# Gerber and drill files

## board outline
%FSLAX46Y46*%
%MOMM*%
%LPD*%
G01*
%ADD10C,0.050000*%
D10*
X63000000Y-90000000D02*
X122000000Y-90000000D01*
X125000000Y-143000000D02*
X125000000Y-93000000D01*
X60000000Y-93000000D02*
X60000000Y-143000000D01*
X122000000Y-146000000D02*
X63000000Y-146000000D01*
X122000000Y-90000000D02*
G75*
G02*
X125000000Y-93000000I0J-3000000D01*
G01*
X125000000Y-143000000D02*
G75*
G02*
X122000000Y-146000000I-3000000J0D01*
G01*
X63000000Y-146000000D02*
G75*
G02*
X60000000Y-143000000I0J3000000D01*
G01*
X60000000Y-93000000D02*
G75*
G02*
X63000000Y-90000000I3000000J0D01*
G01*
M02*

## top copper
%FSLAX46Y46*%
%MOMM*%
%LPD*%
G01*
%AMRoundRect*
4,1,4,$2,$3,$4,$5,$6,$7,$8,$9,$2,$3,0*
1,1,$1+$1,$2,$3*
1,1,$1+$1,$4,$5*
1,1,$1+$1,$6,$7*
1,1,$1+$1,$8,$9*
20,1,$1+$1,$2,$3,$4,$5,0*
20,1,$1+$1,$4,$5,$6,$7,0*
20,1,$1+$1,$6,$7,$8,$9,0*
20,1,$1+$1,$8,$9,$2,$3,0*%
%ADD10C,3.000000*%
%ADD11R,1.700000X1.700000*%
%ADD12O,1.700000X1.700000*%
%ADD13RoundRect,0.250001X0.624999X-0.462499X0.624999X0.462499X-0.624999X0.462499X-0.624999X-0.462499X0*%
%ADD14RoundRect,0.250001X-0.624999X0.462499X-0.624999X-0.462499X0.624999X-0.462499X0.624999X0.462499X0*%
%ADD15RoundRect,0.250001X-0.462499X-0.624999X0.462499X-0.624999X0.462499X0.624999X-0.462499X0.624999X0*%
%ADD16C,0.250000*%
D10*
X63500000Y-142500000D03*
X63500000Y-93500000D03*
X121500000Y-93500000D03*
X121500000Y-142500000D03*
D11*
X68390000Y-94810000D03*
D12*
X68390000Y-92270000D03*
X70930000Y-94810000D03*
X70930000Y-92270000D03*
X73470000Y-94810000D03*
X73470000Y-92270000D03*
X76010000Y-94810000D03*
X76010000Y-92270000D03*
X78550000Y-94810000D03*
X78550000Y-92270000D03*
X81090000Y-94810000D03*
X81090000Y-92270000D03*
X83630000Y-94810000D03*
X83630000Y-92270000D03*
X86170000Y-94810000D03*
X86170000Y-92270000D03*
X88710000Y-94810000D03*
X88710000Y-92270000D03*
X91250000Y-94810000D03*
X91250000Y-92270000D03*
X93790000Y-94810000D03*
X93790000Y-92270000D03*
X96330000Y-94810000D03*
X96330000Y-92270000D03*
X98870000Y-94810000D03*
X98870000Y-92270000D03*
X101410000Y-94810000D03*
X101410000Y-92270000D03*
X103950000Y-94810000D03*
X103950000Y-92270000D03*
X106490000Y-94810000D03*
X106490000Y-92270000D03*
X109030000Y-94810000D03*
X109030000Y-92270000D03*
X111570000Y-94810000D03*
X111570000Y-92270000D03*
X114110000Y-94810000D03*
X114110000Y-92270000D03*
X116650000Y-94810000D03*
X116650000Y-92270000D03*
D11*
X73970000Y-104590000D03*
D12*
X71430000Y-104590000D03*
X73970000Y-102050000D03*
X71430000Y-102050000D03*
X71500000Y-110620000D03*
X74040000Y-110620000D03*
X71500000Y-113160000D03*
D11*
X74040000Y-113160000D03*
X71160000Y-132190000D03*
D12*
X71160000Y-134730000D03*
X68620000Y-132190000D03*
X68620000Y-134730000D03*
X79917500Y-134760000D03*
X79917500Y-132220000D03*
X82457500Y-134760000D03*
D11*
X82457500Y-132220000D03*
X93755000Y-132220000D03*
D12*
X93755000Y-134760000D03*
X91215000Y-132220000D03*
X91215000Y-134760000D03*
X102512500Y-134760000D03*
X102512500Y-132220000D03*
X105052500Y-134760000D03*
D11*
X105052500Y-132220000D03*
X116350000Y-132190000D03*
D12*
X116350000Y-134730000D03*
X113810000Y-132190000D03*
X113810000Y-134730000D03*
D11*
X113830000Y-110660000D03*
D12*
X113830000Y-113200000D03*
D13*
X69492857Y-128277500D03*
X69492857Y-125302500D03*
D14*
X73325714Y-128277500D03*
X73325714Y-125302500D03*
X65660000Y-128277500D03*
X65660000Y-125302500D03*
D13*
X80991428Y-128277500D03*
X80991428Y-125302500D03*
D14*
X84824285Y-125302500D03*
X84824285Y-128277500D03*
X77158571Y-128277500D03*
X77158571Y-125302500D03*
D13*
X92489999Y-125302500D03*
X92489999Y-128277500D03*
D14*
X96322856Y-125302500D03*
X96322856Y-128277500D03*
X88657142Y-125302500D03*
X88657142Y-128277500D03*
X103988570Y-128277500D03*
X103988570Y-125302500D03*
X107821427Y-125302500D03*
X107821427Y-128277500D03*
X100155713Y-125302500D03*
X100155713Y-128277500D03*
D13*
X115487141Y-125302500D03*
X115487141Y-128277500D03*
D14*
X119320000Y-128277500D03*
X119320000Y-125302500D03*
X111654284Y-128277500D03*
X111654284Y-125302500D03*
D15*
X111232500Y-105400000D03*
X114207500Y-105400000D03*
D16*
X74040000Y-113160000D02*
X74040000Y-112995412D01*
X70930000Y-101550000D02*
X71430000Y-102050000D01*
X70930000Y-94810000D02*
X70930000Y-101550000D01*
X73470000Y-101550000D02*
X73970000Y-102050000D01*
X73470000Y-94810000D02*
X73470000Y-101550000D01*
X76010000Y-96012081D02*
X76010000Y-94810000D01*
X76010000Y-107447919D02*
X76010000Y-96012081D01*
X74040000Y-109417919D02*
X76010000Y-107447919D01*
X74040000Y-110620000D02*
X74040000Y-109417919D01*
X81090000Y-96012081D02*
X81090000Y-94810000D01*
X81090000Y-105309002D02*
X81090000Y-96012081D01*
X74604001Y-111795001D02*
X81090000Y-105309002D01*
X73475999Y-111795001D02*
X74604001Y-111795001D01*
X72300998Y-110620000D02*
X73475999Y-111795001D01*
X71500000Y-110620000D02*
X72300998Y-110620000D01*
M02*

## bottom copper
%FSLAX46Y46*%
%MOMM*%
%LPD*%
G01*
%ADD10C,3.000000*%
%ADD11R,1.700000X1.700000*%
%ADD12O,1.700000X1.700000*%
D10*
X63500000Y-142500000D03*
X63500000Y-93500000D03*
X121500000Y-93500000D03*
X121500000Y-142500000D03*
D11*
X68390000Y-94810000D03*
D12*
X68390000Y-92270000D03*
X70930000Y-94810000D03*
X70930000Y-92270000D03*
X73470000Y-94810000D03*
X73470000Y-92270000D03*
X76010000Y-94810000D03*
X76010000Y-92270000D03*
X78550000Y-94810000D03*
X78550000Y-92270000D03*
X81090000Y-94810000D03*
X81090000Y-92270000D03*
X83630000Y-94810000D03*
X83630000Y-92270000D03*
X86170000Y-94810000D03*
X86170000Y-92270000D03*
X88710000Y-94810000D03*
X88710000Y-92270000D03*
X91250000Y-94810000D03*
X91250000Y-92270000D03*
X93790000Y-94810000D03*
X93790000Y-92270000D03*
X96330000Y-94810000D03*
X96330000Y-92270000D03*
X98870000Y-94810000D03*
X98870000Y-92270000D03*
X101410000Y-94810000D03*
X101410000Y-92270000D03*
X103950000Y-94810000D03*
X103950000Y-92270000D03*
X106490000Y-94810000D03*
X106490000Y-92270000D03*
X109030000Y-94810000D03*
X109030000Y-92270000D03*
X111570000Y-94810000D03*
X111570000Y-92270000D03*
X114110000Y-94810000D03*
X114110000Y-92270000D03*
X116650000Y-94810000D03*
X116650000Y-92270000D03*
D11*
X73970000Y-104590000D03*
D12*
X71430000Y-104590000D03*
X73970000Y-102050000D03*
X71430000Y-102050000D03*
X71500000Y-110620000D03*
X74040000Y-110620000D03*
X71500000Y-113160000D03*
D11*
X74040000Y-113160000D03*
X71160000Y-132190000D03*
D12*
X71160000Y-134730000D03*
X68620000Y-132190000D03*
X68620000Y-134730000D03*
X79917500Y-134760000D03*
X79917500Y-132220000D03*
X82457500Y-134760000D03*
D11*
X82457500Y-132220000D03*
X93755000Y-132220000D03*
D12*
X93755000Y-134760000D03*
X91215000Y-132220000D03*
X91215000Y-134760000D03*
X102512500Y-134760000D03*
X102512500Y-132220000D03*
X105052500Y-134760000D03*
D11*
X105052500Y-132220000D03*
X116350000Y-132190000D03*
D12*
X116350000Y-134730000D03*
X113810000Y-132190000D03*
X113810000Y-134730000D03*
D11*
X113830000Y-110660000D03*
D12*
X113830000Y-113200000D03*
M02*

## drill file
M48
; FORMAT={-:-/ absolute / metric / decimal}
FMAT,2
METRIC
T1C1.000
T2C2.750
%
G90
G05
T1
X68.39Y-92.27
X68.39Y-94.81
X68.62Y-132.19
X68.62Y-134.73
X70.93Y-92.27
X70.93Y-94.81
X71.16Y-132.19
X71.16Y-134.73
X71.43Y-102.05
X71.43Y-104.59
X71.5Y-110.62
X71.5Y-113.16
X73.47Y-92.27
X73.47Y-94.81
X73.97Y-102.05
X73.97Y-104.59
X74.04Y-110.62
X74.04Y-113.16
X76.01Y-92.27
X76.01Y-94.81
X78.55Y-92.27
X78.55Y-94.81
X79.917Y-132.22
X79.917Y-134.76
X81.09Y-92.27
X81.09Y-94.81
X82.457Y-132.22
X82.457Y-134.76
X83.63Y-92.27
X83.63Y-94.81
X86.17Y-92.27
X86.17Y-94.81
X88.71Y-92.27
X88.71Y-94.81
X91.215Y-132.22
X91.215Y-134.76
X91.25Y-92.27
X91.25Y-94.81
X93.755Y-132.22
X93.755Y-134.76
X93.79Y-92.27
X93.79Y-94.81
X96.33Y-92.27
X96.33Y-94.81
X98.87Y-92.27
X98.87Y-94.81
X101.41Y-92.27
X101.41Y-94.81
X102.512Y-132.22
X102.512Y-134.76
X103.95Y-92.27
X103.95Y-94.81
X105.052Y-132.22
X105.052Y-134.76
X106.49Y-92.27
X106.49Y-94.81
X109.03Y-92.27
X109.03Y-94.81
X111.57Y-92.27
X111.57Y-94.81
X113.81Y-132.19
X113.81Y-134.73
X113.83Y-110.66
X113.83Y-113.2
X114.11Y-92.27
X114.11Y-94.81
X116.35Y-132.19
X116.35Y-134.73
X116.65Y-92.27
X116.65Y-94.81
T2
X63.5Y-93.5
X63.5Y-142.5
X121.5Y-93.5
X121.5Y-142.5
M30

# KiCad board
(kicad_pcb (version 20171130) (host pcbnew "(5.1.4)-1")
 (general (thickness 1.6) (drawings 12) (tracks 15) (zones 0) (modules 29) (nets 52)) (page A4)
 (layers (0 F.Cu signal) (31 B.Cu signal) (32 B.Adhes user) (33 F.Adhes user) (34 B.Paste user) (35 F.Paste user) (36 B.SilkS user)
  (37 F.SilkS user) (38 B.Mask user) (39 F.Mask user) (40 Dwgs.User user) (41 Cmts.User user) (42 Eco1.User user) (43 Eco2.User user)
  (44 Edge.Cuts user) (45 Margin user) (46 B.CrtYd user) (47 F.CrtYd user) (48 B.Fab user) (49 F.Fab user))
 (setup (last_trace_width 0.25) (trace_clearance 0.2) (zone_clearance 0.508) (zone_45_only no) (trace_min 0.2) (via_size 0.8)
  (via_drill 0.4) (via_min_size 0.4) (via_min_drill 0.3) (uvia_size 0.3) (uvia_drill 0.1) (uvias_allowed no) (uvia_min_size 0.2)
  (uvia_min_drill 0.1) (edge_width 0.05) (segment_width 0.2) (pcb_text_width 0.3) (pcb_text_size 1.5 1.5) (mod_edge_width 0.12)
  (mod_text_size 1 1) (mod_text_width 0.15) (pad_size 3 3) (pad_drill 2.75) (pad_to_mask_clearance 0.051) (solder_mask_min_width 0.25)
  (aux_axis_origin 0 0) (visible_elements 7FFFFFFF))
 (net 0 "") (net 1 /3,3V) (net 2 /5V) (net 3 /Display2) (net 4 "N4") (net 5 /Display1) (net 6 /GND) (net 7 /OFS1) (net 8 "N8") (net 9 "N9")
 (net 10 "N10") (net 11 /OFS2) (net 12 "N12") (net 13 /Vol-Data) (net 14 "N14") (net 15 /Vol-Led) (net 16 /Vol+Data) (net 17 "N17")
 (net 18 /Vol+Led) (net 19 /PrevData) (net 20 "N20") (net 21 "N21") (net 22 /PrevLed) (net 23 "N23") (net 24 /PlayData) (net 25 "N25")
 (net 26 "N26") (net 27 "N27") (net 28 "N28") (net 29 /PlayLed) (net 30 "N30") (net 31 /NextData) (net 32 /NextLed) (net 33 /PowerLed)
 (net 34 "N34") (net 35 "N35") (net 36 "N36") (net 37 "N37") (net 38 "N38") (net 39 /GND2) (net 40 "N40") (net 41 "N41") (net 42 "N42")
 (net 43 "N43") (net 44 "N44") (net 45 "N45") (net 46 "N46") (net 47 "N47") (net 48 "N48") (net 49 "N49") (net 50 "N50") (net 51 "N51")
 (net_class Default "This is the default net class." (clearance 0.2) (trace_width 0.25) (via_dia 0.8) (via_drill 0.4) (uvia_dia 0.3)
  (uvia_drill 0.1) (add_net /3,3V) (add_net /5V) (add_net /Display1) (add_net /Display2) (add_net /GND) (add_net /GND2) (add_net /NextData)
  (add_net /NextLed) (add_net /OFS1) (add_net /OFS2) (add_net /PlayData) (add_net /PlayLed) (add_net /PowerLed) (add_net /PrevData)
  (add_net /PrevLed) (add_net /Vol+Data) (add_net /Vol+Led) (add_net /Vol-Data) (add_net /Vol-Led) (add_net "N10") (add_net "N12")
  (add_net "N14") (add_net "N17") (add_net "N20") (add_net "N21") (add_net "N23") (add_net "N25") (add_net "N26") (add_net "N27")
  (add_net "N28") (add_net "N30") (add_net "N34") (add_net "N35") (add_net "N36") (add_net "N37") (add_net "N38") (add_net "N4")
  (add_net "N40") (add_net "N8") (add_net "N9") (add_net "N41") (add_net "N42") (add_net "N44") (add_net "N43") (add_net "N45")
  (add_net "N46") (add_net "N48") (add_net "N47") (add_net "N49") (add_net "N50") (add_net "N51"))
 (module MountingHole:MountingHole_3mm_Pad (layer F.Cu) (at 63.5 142.5)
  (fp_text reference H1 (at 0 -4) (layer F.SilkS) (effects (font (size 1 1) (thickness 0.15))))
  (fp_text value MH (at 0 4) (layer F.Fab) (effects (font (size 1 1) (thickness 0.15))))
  (pad "" np_thru_hole circle (at 0 0) (size 3 3) (drill 2.75) (layers *.Cu *.Mask)))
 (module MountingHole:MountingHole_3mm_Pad (layer F.Cu) (at 63.5 93.5)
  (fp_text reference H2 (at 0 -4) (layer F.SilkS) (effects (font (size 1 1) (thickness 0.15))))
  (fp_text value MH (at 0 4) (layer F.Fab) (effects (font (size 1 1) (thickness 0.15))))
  (pad "" np_thru_hole circle (at 0 0) (size 3 3) (drill 2.75) (layers *.Cu *.Mask)))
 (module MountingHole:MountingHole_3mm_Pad (layer F.Cu) (at 121.5 93.5)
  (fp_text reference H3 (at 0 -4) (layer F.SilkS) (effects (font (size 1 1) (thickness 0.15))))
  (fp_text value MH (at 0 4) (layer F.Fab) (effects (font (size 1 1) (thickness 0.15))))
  (pad "" np_thru_hole circle (at 0 0) (size 3 3) (drill 2.75) (layers *.Cu *.Mask)))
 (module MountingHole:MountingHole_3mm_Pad (layer F.Cu) (at 121.5 142.5)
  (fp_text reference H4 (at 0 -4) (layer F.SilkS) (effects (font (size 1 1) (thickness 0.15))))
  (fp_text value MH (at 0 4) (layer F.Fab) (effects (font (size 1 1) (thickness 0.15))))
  (pad "" np_thru_hole circle (at 0 0) (size 3 3) (drill 2.75) (layers *.Cu *.Mask)))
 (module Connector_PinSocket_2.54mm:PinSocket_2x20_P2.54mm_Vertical (layer B.Cu) (at 68.39 94.81 270)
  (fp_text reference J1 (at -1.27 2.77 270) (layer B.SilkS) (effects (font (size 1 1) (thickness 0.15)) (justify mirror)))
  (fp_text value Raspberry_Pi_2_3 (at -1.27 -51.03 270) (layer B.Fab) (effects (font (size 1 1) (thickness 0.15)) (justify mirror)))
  (pad 1 thru_hole rect (at 0 0 270) (size 1.7 1.7) (drill 1) (layers *.Cu *.Mask) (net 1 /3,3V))
  (pad 2 thru_hole oval (at -2.54 0 270) (size 1.7 1.7) (drill 1) (layers *.Cu *.Mask) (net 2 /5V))
  (pad 3 thru_hole oval (at 0 -2.54 270) (size 1.7 1.7) (drill 1) (layers *.Cu *.Mask) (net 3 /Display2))
  (pad 4 thru_hole oval (at -2.54 -2.54 270) (size 1.7 1.7) (drill 1) (layers *.Cu *.Mask) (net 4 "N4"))
  (pad 5 thru_hole oval (at 0 -5.08 270) (size 1.7 1.7) (drill 1) (layers *.Cu *.Mask) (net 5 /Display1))
  (pad 6 thru_hole oval (at -2.54 -5.08 270) (size 1.7 1.7) (drill 1) (layers *.Cu *.Mask) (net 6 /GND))
  (pad 7 thru_hole oval (at 0 -7.62 270) (size 1.7 1.7) (drill 1) (layers *.Cu *.Mask) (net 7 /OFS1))
  (pad 8 thru_hole oval (at -2.54 -7.62 270) (size 1.7 1.7) (drill 1) (layers *.Cu *.Mask) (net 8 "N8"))
  (pad 9 thru_hole oval (at 0 -10.16 270) (size 1.7 1.7) (drill 1) (layers *.Cu *.Mask) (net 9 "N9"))
  (pad 10 thru_hole oval (at -2.54 -10.16 270) (size 1.7 1.7) (drill 1) (layers *.Cu *.Mask) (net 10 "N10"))
  (pad 11 thru_hole oval (at 0 -12.7 270) (size 1.7 1.7) (drill 1) (layers *.Cu *.Mask) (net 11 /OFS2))
  (pad 12 thru_hole oval (at -2.54 -12.7 270) (size 1.7 1.7) (drill 1) (layers *.Cu *.Mask) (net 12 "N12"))
  (pad 13 thru_hole oval (at 0 -15.24 270) (size 1.7 1.7) (drill 1) (layers *.Cu *.Mask) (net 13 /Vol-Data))
  (pad 14 thru_hole oval (at -2.54 -15.24 270) (size 1.7 1.7) (drill 1) (layers *.Cu *.Mask) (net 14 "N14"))
  (pad 15 thru_hole oval (at 0 -17.78 270) (size 1.7 1.7) (drill 1) (layers *.Cu *.Mask) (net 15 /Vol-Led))
  (pad 16 thru_hole oval (at -2.54 -17.78 270) (size 1.7 1.7) (drill 1) (layers *.Cu *.Mask) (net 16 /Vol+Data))
  (pad 17 thru_hole oval (at 0 -20.32 270) (size 1.7 1.7) (drill 1) (layers *.Cu *.Mask) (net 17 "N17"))
  (pad 18 thru_hole oval (at -2.54 -20.32 270) (size 1.7 1.7) (drill 1) (layers *.Cu *.Mask) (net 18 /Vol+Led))
  (pad 19 thru_hole oval (at 0 -22.86 270) (size 1.7 1.7) (drill 1) (layers *.Cu *.Mask) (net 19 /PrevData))
  (pad 20 thru_hole oval (at -2.54 -22.86 270) (size 1.7 1.7) (drill 1) (layers *.Cu *.Mask) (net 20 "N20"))
  (pad 21 thru_hole oval (at 0 -25.4 270) (size 1.7 1.7) (drill 1) (layers *.Cu *.Mask) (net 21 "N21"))
  (pad 22 thru_hole oval (at -2.54 -25.4 270) (size 1.7 1.7) (drill 1) (layers *.Cu *.Mask) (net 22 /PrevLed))
  (pad 23 thru_hole oval (at 0 -27.94 270) (size 1.7 1.7) (drill 1) (layers *.Cu *.Mask) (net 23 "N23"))
  (pad 24 thru_hole oval (at -2.54 -27.94 270) (size 1.7 1.7) (drill 1) (layers *.Cu *.Mask) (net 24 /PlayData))
  (pad 25 thru_hole oval (at 0 -30.48 270) (size 1.7 1.7) (drill 1) (layers *.Cu *.Mask) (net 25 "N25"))
  (pad 26 thru_hole oval (at -2.54 -30.48 270) (size 1.7 1.7) (drill 1) (layers *.Cu *.Mask) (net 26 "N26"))
  (pad 27 thru_hole oval (at 0 -33.02 270) (size 1.7 1.7) (drill 1) (layers *.Cu *.Mask) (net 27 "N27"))
  (pad 28 thru_hole oval (at -2.54 -33.02 270) (size 1.7 1.7) (drill 1) (layers *.Cu *.Mask) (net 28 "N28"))
  (pad 29 thru_hole oval (at 0 -35.56 270) (size 1.7 1.7) (drill 1) (layers *.Cu *.Mask) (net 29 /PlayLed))
  (pad 30 thru_hole oval (at -2.54 -35.56 270) (size 1.7 1.7) (drill 1) (layers *.Cu *.Mask) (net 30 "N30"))
  (pad 31 thru_hole oval (at 0 -38.1 270) (size 1.7 1.7) (drill 1) (layers *.Cu *.Mask) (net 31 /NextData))
  (pad 32 thru_hole oval (at -2.54 -38.1 270) (size 1.7 1.7) (drill 1) (layers *.Cu *.Mask) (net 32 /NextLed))
  (pad 33 thru_hole oval (at 0 -40.64 270) (size 1.7 1.7) (drill 1) (layers *.Cu *.Mask) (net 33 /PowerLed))
  (pad 34 thru_hole oval (at -2.54 -40.64 270) (size 1.7 1.7) (drill 1) (layers *.Cu *.Mask) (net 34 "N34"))
  (pad 35 thru_hole oval (at 0 -43.18 270) (size 1.7 1.7) (drill 1) (layers *.Cu *.Mask) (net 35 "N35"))
  (pad 36 thru_hole oval (at -2.54 -43.18 270) (size 1.7 1.7) (drill 1) (layers *.Cu *.Mask) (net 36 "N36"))
  (pad 37 thru_hole oval (at 0 -45.72 270) (size 1.7 1.7) (drill 1) (layers *.Cu *.Mask) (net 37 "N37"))
  (pad 38 thru_hole oval (at -2.54 -45.72 270) (size 1.7 1.7) (drill 1) (layers *.Cu *.Mask) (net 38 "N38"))
  (pad 39 thru_hole oval (at 0 -48.26 270) (size 1.7 1.7) (drill 1) (layers *.Cu *.Mask) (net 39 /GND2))
  (pad 40 thru_hole oval (at -2.54 -48.26 270) (size 1.7 1.7) (drill 1) (layers *.Cu *.Mask) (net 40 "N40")))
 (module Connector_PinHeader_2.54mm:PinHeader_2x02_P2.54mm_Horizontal (layer F.Cu) (at 73.97 104.59 180)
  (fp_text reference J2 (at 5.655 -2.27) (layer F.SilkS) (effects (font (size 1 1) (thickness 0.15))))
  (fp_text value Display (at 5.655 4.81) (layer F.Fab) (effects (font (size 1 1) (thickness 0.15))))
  (pad 1 thru_hole rect (at 0 0 180) (size 1.7 1.7) (drill 1) (layers *.Cu *.Mask) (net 2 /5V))
  (pad 2 thru_hole oval (at 2.54 0 180) (size 1.7 1.7) (drill 1) (layers *.Cu *.Mask) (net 6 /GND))
  (pad 3 thru_hole oval (at 0 2.54 180) (size 1.7 1.7) (drill 1) (layers *.Cu *.Mask) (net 5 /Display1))
  (pad 4 thru_hole oval (at 2.54 2.54 180) (size 1.7 1.7) (drill 1) (layers *.Cu *.Mask) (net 3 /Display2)))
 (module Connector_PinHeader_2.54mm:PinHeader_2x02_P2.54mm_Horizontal (layer F.Cu) (at 74.04 113.16 180)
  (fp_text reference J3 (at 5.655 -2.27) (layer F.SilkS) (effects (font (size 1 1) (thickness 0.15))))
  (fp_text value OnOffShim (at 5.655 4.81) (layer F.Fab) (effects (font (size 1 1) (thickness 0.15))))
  (pad 4 thru_hole oval (at 2.54 2.54 180) (size 1.7 1.7) (drill 1) (layers *.Cu *.Mask) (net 11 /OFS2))
  (pad 3 thru_hole oval (at 0 2.54 180) (size 1.7 1.7) (drill 1) (layers *.Cu *.Mask) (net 7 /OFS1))
  (pad 2 thru_hole oval (at 2.54 0 180) (size 1.7 1.7) (drill 1) (layers *.Cu *.Mask) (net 6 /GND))
  (pad 1 thru_hole rect (at 0 0 180) (size 1.7 1.7) (drill 1) (layers *.Cu *.Mask) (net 2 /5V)))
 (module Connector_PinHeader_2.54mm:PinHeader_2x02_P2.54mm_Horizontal (layer F.Cu) (at 71.16 132.19 270)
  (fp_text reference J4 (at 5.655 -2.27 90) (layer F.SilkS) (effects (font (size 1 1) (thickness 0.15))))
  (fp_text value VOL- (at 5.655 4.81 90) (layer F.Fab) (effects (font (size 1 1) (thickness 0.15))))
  (pad 1 thru_hole rect (at 0 0 270) (size 1.7 1.7) (drill 1) (layers *.Cu *.Mask) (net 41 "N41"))
  (pad 2 thru_hole oval (at 2.54 0 270) (size 1.7 1.7) (drill 1) (layers *.Cu *.Mask) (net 6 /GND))
  (pad 3 thru_hole oval (at 0 2.54 270) (size 1.7 1.7) (drill 1) (layers *.Cu *.Mask) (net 6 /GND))
  (pad 4 thru_hole oval (at 2.54 2.54 270) (size 1.7 1.7) (drill 1) (layers *.Cu *.Mask) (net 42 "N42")))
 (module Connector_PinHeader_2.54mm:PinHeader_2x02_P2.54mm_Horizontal (layer F.Cu) (at 82.4575 132.22 270)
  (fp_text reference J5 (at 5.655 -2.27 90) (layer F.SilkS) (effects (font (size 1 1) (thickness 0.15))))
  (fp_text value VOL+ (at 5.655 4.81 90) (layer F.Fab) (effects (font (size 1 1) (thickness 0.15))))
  (pad 4 thru_hole oval (at 2.54 2.54 270) (size 1.7 1.7) (drill 1) (layers *.Cu *.Mask) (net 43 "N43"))
  (pad 3 thru_hole oval (at 0 2.54 270) (size 1.7 1.7) (drill 1) (layers *.Cu *.Mask) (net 6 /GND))
  (pad 2 thru_hole oval (at 2.54 0 270) (size 1.7 1.7) (drill 1) (layers *.Cu *.Mask) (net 6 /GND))
  (pad 1 thru_hole rect (at 0 0 270) (size 1.7 1.7) (drill 1) (layers *.Cu *.Mask) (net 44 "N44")))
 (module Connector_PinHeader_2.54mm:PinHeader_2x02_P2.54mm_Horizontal (layer F.Cu) (at 93.755 132.22 270)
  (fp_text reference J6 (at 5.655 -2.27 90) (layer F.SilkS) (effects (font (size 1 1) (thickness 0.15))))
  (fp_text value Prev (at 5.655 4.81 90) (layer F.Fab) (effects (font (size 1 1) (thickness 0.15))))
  (pad 1 thru_hole rect (at 0 0 270) (size 1.7 1.7) (drill 1) (layers *.Cu *.Mask) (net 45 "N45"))
  (pad 2 thru_hole oval (at 2.54 0 270) (size 1.7 1.7) (drill 1) (layers *.Cu *.Mask) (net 39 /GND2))
  (pad 3 thru_hole oval (at 0 2.54 270) (size 1.7 1.7) (drill 1) (layers *.Cu *.Mask) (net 39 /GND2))
  (pad 4 thru_hole oval (at 2.54 2.54 270) (size 1.7 1.7) (drill 1) (layers *.Cu *.Mask) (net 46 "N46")))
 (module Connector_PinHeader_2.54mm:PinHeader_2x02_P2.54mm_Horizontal (layer F.Cu) (at 105.0525 132.22 270)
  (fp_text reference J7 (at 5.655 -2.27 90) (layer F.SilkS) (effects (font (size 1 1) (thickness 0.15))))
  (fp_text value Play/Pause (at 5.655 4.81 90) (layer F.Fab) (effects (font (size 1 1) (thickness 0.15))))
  (pad 4 thru_hole oval (at 2.54 2.54 270) (size 1.7 1.7) (drill 1) (layers *.Cu *.Mask) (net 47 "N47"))
  (pad 3 thru_hole oval (at 0 2.54 270) (size 1.7 1.7) (drill 1) (layers *.Cu *.Mask) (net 39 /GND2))
  (pad 2 thru_hole oval (at 2.54 0 270) (size 1.7 1.7) (drill 1) (layers *.Cu *.Mask) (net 39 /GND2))
  (pad 1 thru_hole rect (at 0 0 270) (size 1.7 1.7) (drill 1) (layers *.Cu *.Mask) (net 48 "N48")))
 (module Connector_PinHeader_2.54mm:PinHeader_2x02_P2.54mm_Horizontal (layer F.Cu) (at 116.35 132.19 270)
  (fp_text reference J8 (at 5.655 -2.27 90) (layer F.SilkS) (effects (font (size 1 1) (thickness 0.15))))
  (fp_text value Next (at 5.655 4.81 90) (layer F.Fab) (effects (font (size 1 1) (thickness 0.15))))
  (pad 1 thru_hole rect (at 0 0 270) (size 1.7 1.7) (drill 1) (layers *.Cu *.Mask) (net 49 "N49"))
  (pad 2 thru_hole oval (at 2.54 0 270) (size 1.7 1.7) (drill 1) (layers *.Cu *.Mask) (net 39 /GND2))
  (pad 3 thru_hole oval (at 0 2.54 270) (size 1.7 1.7) (drill 1) (layers *.Cu *.Mask) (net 39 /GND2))
  (pad 4 thru_hole oval (at 2.54 2.54 270) (size 1.7 1.7) (drill 1) (layers *.Cu *.Mask) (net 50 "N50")))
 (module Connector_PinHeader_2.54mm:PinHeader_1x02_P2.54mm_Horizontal (layer F.Cu) (at 113.83 110.66)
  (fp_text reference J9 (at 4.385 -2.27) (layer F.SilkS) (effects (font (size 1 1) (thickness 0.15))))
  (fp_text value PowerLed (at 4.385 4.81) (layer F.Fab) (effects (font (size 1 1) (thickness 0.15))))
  (pad 1 thru_hole rect (at 0 0) (size 1.7 1.7) (drill 1) (layers *.Cu *.Mask) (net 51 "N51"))
  (pad 2 thru_hole oval (at 0 2.54) (size 1.7 1.7) (drill 1) (layers *.Cu *.Mask) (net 39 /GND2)))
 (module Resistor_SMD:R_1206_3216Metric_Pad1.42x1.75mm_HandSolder (layer F.Cu) (at 69.492857 126.79 90)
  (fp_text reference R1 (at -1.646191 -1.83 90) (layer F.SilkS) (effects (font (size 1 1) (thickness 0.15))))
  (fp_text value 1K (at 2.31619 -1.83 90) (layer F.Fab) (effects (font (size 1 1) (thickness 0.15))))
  (pad 1 smd roundrect (at -1.4875 0 90) (size 1.425 1.75) (layers F.Cu F.Paste F.Mask) (roundrect_rratio 0.175439) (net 41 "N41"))
  (pad 2 smd roundrect (at 1.4875 0 90) (size 1.425 1.75) (layers F.Cu F.Paste F.Mask) (roundrect_rratio 0.175439) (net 13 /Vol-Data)))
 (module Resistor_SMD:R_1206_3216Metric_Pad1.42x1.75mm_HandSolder (layer F.Cu) (at 73.325714 126.79 270)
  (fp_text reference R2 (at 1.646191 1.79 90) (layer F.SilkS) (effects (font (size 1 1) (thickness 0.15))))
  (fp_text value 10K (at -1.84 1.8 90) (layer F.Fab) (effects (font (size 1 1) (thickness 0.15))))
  (pad 2 smd roundrect (at 1.4875 0 270) (size 1.425 1.75) (layers F.Cu F.Paste F.Mask) (roundrect_rratio 0.175439) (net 41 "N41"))
  (pad 1 smd roundrect (at -1.4875 0 270) (size 1.425 1.75) (layers F.Cu F.Paste F.Mask) (roundrect_rratio 0.175439) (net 1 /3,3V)))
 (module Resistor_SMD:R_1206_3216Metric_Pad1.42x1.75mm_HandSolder (layer F.Cu) (at 65.66 126.79 270)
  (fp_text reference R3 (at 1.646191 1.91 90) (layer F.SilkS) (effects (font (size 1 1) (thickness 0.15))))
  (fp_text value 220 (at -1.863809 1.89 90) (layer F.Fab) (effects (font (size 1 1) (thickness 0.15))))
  (pad 2 smd roundrect (at 1.4875 0 270) (size 1.425 1.75) (layers F.Cu F.Paste F.Mask) (roundrect_rratio 0.175439) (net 42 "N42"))
  (pad 1 smd roundrect (at -1.4875 0 270) (size 1.425 1.75) (layers F.Cu F.Paste F.Mask) (roundrect_rratio 0.175439) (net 15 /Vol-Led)))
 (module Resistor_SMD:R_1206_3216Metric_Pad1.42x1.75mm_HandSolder (layer F.Cu) (at 80.991428 126.79 90)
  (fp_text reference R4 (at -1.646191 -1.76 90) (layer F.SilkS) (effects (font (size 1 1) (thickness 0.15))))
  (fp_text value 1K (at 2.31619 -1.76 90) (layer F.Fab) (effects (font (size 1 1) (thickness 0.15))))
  (pad 1 smd roundrect (at -1.4875 0 90) (size 1.425 1.75) (layers F.Cu F.Paste F.Mask) (roundrect_rratio 0.175439) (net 44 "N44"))
  (pad 2 smd roundrect (at 1.4875 0 90) (size 1.425 1.75) (layers F.Cu F.Paste F.Mask) (roundrect_rratio 0.175439) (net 16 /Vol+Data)))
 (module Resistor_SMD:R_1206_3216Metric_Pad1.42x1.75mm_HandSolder (layer F.Cu) (at 84.824285 126.79 270)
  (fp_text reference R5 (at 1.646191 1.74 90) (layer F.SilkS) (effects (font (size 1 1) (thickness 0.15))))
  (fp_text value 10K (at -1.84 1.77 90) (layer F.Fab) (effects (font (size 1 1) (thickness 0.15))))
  (pad 1 smd roundrect (at -1.4875 0 270) (size 1.425 1.75) (layers F.Cu F.Paste F.Mask) (roundrect_rratio 0.175439) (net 1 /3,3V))
  (pad 2 smd roundrect (at 1.4875 0 270) (size 1.425 1.75) (layers F.Cu F.Paste F.Mask) (roundrect_rratio 0.175439) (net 44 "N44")))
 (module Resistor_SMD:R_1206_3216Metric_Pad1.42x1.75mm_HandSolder (layer F.Cu) (at 77.158571 126.79 270)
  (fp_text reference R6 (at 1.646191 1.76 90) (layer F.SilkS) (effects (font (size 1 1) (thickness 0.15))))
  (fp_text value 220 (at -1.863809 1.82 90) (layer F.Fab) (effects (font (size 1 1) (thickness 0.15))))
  (pad 2 smd roundrect (at 1.4875 0 270) (size 1.425 1.75) (layers F.Cu F.Paste F.Mask) (roundrect_rratio 0.175439) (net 43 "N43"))
  (pad 1 smd roundrect (at -1.4875 0 270) (size 1.425 1.75) (layers F.Cu F.Paste F.Mask) (roundrect_rratio 0.175439) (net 18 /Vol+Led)))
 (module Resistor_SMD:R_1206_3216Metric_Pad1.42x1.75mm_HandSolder (layer F.Cu) (at 92.489999 126.79 90)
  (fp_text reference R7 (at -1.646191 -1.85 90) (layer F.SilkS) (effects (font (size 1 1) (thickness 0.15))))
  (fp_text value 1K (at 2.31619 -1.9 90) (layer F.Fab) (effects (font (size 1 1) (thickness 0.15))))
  (pad 2 smd roundrect (at 1.4875 0 90) (size 1.425 1.75) (layers F.Cu F.Paste F.Mask) (roundrect_rratio 0.175439) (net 19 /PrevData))
  (pad 1 smd roundrect (at -1.4875 0 90) (size 1.425 1.75) (layers F.Cu F.Paste F.Mask) (roundrect_rratio 0.175439) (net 45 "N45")))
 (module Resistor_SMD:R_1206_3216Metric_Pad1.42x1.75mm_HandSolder (layer F.Cu) (at 96.322856 126.79 270)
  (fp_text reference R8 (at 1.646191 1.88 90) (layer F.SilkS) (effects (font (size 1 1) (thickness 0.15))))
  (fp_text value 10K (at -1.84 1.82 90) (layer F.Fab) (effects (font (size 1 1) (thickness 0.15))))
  (pad 1 smd roundrect (at -1.4875 0 270) (size 1.425 1.75) (layers F.Cu F.Paste F.Mask) (roundrect_rratio 0.175439) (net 1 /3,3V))
  (pad 2 smd roundrect (at 1.4875 0 270) (size 1.425 1.75) (layers F.Cu F.Paste F.Mask) (roundrect_rratio 0.175439) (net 45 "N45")))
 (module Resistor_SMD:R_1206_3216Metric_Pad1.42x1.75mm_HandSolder (layer F.Cu) (at 88.657142 126.79 270)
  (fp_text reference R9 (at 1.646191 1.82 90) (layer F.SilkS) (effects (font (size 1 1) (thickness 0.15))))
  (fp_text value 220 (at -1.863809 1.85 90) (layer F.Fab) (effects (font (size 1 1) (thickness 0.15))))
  (pad 1 smd roundrect (at -1.4875 0 270) (size 1.425 1.75) (layers F.Cu F.Paste F.Mask) (roundrect_rratio 0.175439) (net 22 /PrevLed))
  (pad 2 smd roundrect (at 1.4875 0 270) (size 1.425 1.75) (layers F.Cu F.Paste F.Mask) (roundrect_rratio 0.175439) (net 46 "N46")))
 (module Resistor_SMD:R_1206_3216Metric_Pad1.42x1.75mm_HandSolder (layer F.Cu) (at 103.98857 126.79 270)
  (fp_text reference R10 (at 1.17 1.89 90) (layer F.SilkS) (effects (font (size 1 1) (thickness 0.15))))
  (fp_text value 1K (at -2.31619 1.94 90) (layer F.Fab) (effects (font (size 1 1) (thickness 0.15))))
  (pad 2 smd roundrect (at 1.4875 0 270) (size 1.425 1.75) (layers F.Cu F.Paste F.Mask) (roundrect_rratio 0.175439) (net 24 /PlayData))
  (pad 1 smd roundrect (at -1.4875 0 270) (size 1.425 1.75) (layers F.Cu F.Paste F.Mask) (roundrect_rratio 0.175439) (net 48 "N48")))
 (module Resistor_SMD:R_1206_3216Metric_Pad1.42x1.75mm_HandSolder (layer F.Cu) (at 107.821427 126.79 270)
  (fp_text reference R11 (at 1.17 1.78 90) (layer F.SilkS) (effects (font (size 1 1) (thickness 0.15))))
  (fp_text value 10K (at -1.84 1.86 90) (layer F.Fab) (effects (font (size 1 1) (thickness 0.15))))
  (pad 1 smd roundrect (at -1.4875 0 270) (size 1.425 1.75) (layers F.Cu F.Paste F.Mask) (roundrect_rratio 0.175439) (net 1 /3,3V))
  (pad 2 smd roundrect (at 1.4875 0 270) (size 1.425 1.75) (layers F.Cu F.Paste F.Mask) (roundrect_rratio 0.175439) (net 48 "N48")))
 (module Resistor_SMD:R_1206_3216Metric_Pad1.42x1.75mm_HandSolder (layer F.Cu) (at 100.155713 126.79 270)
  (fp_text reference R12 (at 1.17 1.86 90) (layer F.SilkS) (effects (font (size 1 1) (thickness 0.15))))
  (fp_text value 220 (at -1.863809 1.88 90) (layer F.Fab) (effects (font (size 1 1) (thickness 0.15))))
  (pad 1 smd roundrect (at -1.4875 0 270) (size 1.425 1.75) (layers F.Cu F.Paste F.Mask) (roundrect_rratio 0.175439) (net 29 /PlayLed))
  (pad 2 smd roundrect (at 1.4875 0 270) (size 1.425 1.75) (layers F.Cu F.Paste F.Mask) (roundrect_rratio 0.175439) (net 47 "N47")))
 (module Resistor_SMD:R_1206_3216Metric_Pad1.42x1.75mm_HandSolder (layer F.Cu) (at 115.487141 126.79 90)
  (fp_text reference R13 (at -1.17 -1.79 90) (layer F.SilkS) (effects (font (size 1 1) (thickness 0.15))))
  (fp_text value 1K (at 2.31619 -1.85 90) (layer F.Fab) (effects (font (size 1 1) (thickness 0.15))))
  (pad 2 smd roundrect (at 1.4875 0 90) (size 1.425 1.75) (layers F.Cu F.Paste F.Mask) (roundrect_rratio 0.175439) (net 31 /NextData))
  (pad 1 smd roundrect (at -1.4875 0 90) (size 1.425 1.75) (layers F.Cu F.Paste F.Mask) (roundrect_rratio 0.175439) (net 49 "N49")))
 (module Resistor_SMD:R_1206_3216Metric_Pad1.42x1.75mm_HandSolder (layer F.Cu) (at 119.32 126.79 270)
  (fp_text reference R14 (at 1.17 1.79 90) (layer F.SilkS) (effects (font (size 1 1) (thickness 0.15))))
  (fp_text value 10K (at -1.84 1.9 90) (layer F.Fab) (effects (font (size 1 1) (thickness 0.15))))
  (pad 2 smd roundrect (at 1.4875 0 270) (size 1.425 1.75) (layers F.Cu F.Paste F.Mask) (roundrect_rratio 0.175439) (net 49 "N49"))
  (pad 1 smd roundrect (at -1.4875 0 270) (size 1.425 1.75) (layers F.Cu F.Paste F.Mask) (roundrect_rratio 0.175439) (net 1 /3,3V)))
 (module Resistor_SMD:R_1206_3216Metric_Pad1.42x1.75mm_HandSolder (layer F.Cu) (at 111.654284 126.79 270)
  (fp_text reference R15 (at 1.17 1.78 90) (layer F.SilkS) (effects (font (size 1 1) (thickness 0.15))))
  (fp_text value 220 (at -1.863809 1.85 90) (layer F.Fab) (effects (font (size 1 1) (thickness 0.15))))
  (pad 2 smd roundrect (at 1.4875 0 270) (size 1.425 1.75) (layers F.Cu F.Paste F.Mask) (roundrect_rratio 0.175439) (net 50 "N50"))
  (pad 1 smd roundrect (at -1.4875 0 270) (size 1.425 1.75) (layers F.Cu F.Paste F.Mask) (roundrect_rratio 0.175439) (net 32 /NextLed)))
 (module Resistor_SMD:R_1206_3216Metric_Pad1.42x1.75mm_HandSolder (layer F.Cu) (at 112.72 105.4)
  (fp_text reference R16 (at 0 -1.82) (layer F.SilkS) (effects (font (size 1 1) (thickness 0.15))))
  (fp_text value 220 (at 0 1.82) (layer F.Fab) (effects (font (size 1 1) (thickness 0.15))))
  (pad 1 smd roundrect (at -1.4875 0) (size 1.425 1.75) (layers F.Cu F.Paste F.Mask) (roundrect_rratio 0.175439) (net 33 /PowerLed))
  (pad 2 smd roundrect (at 1.4875 0) (size 1.425 1.75) (layers F.Cu F.Paste F.Mask) (roundrect_rratio 0.175439) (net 51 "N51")))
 (gr_line (start 63 90) (end 122 90) (layer Edge.Cuts) (width 0.05))
 (gr_line (start 125 143) (end 125 93) (layer Edge.Cuts) (width 0.05))
 (gr_line (start 60 93) (end 60 143) (layer Edge.Cuts) (width 0.05))
 (gr_line (start 122 146) (end 63 146) (layer Edge.Cuts) (width 0.05))
 (gr_arc (start 122 93) (end 125 93) (angle -90) (layer Edge.Cuts) (width 0.05))
 (gr_arc (start 122 143) (end 122 146) (angle -90) (layer Edge.Cuts) (width 0.05))
 (gr_arc (start 63 143) (end 60 143) (angle -90) (layer Edge.Cuts) (width 0.05))
 (gr_arc (start 63 93) (end 63 90) (angle -90) (layer Edge.Cuts) (width 0.05))
 (segment (start 74.04 113.16) (end 74.04 112.995412) (width 0.25) (layer F.Cu) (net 2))
 (segment (start 70.93 101.55) (end 71.43 102.05) (width 0.25) (layer F.Cu) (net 3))
 (segment (start 70.93 94.81) (end 70.93 101.55) (width 0.25) (layer F.Cu) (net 3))
 (segment (start 73.47 101.55) (end 73.97 102.05) (width 0.25) (layer F.Cu) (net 5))
 (segment (start 73.47 94.81) (end 73.47 101.55) (width 0.25) (layer F.Cu) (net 5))
 (segment (start 76.01 96.012081) (end 76.01 94.81) (width 0.25) (layer F.Cu) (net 7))
 (segment (start 76.01 107.447919) (end 76.01 96.012081) (width 0.25) (layer F.Cu) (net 7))
 (segment (start 74.04 109.417919) (end 76.01 107.447919) (width 0.25) (layer F.Cu) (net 7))
 (segment (start 74.04 110.62) (end 74.04 109.417919) (width 0.25) (layer F.Cu) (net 7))
 (segment (start 81.09 96.012081) (end 81.09 94.81) (width 0.25) (layer F.Cu) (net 11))
 (segment (start 81.09 105.309002) (end 81.09 96.012081) (width 0.25) (layer F.Cu) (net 11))
 (segment (start 74.604001 111.795001) (end 81.09 105.309002) (width 0.25) (layer F.Cu) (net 11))
 (segment (start 73.475999 111.795001) (end 74.604001 111.795001) (width 0.25) (layer F.Cu) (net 11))
 (segment (start 72.300998 110.62) (end 73.475999 111.795001) (width 0.25) (layer F.Cu) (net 11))
 (segment (start 71.5 110.62) (end 72.300998 110.62) (width 0.25) (layer F.Cu) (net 11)))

